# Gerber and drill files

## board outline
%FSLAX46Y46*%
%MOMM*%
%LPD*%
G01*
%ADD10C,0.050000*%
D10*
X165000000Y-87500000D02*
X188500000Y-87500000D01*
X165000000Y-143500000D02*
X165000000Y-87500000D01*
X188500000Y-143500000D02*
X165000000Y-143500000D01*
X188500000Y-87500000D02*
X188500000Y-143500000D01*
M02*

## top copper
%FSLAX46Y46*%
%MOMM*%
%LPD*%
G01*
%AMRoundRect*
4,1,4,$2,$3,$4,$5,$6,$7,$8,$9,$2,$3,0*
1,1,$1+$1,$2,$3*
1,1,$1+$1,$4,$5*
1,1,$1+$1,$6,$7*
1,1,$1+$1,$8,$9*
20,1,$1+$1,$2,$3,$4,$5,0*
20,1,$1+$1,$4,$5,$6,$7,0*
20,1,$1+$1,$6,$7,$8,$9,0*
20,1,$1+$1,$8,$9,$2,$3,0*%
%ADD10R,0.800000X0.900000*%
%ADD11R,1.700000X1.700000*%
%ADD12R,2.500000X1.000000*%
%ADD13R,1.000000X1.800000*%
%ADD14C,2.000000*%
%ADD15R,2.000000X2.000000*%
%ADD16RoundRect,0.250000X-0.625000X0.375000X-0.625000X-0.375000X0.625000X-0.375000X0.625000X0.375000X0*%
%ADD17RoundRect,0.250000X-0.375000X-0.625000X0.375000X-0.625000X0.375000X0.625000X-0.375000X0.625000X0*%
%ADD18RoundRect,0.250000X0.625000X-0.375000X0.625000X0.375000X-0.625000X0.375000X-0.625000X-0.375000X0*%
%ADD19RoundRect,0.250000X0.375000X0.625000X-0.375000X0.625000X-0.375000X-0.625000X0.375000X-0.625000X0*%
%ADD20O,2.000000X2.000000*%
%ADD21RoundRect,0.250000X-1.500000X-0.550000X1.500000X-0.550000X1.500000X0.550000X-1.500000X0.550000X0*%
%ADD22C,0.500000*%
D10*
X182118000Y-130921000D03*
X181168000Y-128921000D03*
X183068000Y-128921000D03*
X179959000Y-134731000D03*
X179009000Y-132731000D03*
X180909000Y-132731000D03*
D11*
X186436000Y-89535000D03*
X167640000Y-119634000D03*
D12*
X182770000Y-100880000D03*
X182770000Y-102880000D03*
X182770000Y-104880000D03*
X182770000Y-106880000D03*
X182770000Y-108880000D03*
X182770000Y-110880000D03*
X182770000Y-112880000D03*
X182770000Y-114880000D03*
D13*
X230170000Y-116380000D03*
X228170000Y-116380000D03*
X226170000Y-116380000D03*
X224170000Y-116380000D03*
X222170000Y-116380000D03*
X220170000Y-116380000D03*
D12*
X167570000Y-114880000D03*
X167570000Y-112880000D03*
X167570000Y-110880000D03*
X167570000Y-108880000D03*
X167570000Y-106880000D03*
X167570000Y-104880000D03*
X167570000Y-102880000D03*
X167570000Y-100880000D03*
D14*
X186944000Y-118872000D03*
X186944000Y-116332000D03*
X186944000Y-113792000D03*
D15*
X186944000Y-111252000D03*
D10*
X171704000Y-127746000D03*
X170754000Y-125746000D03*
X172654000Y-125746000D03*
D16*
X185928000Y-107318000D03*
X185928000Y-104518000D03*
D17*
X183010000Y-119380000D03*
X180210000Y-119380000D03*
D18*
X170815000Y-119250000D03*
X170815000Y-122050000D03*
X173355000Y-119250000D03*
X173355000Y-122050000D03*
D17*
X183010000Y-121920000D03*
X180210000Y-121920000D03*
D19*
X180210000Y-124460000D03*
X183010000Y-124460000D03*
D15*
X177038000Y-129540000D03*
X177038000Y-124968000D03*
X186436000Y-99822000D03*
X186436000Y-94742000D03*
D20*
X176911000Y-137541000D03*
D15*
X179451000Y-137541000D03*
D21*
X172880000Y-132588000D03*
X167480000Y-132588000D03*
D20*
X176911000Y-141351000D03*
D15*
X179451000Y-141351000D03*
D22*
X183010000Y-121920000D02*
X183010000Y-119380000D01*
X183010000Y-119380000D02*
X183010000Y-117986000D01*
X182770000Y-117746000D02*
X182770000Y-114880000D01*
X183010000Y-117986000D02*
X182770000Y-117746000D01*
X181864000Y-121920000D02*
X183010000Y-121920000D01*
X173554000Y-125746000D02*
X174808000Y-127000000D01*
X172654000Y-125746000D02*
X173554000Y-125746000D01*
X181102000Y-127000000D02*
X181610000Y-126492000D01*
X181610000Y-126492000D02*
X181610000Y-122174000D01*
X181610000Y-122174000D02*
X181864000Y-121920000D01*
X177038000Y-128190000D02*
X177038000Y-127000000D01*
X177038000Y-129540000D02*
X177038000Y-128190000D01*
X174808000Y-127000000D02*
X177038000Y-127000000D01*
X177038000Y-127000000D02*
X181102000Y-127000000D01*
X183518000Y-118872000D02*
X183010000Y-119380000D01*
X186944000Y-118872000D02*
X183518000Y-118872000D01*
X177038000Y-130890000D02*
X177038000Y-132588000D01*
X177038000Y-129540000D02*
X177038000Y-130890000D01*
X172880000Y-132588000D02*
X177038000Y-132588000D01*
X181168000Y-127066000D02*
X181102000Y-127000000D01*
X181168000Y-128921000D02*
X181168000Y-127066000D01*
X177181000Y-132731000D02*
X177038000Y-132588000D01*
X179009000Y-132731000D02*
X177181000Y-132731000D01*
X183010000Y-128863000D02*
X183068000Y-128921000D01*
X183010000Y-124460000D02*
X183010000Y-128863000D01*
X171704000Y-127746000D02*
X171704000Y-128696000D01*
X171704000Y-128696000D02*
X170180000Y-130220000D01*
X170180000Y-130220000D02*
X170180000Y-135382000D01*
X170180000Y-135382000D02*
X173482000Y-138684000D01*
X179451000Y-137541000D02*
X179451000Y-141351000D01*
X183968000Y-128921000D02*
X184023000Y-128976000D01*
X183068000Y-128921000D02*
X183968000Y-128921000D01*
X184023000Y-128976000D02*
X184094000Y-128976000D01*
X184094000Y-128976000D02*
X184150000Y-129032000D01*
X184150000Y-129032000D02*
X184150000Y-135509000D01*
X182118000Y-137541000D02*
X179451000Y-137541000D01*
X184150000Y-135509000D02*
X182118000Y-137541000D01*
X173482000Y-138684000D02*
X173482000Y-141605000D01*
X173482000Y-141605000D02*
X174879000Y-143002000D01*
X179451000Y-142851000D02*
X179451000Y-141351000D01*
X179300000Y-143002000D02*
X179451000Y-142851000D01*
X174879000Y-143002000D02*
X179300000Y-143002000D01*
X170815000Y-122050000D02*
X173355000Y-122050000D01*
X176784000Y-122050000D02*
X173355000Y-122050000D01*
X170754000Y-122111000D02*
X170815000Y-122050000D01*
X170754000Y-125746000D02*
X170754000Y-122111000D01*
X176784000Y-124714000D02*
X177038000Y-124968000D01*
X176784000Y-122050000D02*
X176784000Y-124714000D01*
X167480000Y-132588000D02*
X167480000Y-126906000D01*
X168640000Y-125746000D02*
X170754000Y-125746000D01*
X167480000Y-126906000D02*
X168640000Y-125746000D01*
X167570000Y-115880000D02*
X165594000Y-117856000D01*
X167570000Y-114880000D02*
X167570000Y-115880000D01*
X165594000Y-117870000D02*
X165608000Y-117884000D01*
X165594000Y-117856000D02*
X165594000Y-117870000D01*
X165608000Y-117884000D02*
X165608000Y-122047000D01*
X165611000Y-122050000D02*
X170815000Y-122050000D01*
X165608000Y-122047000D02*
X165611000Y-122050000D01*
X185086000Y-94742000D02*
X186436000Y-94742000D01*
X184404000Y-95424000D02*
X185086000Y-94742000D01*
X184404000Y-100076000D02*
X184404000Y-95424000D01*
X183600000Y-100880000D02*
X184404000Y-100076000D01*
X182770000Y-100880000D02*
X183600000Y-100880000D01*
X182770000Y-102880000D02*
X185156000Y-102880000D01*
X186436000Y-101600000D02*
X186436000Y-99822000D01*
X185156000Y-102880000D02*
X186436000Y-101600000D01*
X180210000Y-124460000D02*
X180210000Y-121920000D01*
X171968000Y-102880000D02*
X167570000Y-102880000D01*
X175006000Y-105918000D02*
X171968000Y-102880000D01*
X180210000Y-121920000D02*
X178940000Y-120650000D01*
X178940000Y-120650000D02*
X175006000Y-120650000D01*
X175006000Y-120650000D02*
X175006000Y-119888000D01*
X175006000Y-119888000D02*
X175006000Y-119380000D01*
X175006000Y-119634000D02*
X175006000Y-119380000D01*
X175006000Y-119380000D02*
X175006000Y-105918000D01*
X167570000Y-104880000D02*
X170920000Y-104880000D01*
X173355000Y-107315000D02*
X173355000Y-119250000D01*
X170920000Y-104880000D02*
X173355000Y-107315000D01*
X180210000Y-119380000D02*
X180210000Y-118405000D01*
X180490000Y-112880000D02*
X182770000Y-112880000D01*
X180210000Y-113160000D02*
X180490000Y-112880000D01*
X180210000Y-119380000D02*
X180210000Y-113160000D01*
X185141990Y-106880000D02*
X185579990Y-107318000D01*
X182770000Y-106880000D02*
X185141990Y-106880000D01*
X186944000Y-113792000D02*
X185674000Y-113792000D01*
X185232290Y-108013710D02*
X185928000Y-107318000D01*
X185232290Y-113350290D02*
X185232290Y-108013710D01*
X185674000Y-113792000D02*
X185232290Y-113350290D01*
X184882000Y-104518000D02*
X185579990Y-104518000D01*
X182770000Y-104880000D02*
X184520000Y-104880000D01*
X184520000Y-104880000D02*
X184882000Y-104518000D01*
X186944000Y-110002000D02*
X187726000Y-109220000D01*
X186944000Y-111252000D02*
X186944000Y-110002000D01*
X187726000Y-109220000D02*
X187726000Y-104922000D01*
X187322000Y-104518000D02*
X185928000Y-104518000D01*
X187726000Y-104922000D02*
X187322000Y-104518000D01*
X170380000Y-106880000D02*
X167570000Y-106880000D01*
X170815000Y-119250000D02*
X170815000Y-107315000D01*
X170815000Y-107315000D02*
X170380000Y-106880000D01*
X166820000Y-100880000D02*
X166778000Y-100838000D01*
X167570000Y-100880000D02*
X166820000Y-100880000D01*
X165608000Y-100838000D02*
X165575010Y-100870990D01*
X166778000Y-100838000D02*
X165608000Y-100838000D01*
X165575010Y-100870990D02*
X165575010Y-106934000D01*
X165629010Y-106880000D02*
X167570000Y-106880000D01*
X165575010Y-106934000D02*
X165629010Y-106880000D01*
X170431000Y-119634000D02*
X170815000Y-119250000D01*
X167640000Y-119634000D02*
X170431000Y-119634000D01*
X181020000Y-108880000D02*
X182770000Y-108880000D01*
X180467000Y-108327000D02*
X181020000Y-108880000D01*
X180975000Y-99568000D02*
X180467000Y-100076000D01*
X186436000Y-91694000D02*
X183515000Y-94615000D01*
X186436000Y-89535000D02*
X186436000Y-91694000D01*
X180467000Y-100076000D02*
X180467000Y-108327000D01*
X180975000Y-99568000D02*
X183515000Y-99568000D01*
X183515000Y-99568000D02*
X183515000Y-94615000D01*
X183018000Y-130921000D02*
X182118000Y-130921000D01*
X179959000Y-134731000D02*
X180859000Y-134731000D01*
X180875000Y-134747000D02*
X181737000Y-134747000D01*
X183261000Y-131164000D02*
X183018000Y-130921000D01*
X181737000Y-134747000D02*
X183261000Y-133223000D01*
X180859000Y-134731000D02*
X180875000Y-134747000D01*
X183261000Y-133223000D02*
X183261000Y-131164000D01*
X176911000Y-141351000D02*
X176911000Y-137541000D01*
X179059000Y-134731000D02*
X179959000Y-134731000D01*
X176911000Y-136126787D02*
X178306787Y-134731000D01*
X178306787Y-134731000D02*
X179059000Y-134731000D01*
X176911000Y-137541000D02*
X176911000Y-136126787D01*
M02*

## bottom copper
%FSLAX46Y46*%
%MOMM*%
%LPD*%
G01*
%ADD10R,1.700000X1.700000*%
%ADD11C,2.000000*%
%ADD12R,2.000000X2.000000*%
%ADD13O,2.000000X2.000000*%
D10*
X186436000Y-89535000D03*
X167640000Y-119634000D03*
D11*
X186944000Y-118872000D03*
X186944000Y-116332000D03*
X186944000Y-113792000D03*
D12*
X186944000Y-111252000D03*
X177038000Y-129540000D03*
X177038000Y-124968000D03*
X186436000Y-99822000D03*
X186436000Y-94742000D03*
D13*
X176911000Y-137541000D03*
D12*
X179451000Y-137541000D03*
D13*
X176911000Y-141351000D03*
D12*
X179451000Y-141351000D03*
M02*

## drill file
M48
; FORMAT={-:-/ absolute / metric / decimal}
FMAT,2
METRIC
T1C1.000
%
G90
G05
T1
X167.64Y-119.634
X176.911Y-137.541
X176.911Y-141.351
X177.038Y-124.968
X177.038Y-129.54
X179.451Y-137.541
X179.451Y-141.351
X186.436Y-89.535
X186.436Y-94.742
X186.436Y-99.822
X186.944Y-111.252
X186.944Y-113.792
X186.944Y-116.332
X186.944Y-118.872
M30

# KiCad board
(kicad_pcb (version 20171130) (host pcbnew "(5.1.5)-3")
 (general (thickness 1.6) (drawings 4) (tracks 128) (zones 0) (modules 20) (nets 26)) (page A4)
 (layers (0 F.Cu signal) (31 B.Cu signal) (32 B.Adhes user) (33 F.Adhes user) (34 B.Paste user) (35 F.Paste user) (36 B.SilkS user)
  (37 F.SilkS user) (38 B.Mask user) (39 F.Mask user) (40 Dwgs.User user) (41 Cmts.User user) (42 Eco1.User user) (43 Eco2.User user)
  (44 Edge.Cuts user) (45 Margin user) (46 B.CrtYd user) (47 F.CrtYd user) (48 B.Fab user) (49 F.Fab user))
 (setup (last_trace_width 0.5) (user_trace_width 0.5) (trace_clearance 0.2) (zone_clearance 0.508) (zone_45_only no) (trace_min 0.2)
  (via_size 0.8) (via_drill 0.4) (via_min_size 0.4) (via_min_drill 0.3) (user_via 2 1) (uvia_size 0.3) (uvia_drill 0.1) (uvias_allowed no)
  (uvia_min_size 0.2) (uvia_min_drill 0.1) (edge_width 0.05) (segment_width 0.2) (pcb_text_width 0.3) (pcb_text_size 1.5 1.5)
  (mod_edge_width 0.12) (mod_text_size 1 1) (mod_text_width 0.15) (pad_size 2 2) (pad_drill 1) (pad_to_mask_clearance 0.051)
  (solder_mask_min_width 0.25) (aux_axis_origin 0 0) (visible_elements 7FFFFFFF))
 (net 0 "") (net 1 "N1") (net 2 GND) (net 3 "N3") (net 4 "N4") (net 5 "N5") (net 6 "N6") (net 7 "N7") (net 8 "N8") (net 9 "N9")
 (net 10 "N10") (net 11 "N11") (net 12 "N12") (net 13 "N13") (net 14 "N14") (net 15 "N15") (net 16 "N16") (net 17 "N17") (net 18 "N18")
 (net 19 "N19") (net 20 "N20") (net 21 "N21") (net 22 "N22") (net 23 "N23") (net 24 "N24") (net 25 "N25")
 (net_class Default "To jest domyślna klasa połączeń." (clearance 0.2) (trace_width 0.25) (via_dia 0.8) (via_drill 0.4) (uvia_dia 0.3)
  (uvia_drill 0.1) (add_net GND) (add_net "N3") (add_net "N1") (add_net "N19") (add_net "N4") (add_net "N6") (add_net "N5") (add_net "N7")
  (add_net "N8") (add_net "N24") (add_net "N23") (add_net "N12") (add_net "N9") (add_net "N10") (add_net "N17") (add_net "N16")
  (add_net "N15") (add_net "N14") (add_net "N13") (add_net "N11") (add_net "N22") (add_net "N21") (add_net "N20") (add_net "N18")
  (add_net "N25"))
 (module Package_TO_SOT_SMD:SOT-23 (layer F.Cu) (at 182.118 129.921 270)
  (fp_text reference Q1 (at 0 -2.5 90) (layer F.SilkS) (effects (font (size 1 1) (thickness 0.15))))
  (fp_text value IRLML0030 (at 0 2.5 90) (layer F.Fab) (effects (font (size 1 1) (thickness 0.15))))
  (pad 3 smd rect (at 1 0 270) (size 0.9 0.8) (layers F.Cu F.Paste F.Mask) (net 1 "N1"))
  (pad 2 smd rect (at -1 0.95 270) (size 0.9 0.8) (layers F.Cu F.Paste F.Mask) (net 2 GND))
  (pad 1 smd rect (at -1 -0.95 270) (size 0.9 0.8) (layers F.Cu F.Paste F.Mask) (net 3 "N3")))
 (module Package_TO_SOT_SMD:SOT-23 (layer F.Cu) (at 179.959 133.731 270)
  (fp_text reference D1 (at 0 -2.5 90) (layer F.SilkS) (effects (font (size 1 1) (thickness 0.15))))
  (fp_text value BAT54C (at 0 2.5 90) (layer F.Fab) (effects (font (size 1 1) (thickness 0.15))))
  (pad 3 smd rect (at 1 0 270) (size 0.9 0.8) (layers F.Cu F.Paste F.Mask) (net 1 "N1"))
  (pad 2 smd rect (at -1 0.95 270) (size 0.9 0.8) (layers F.Cu F.Paste F.Mask) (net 2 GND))
  (pad 1 smd rect (at -1 -0.95 270) (size 0.9 0.8) (layers F.Cu F.Paste F.Mask) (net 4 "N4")))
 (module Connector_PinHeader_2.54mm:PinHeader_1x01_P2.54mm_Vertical (layer F.Cu) (at 186.436 89.535)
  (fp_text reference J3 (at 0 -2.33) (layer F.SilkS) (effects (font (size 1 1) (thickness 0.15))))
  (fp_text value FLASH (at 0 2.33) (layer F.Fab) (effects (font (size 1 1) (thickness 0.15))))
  (pad 1 thru_hole rect (at 0 0) (size 1.7 1.7) (drill 1) (layers *.Cu *.Mask) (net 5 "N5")))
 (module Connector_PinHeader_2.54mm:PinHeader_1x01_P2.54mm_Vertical (layer F.Cu) (at 167.64 119.634)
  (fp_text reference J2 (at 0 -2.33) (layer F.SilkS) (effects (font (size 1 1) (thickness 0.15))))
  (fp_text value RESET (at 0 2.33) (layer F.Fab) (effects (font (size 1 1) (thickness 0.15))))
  (pad 1 thru_hole rect (at 0 0) (size 1.7 1.7) (drill 1) (layers *.Cu *.Mask) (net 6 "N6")))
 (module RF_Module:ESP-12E (layer F.Cu) (at 175.17 104.38)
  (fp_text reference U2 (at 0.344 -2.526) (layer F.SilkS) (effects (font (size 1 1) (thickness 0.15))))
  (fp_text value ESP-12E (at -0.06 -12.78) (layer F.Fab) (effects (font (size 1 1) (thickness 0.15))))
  (pad 22 smd rect (at 7.6 -3.5) (size 2.5 1) (layers F.Cu F.Paste F.Mask) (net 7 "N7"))
  (pad 21 smd rect (at 7.6 -1.5) (size 2.5 1) (layers F.Cu F.Paste F.Mask) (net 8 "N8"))
  (pad 20 smd rect (at 7.6 0.5) (size 2.5 1) (layers F.Cu F.Paste F.Mask) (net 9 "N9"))
  (pad 19 smd rect (at 7.6 2.5) (size 2.5 1) (layers F.Cu F.Paste F.Mask) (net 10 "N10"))
  (pad 18 smd rect (at 7.6 4.5) (size 2.5 1) (layers F.Cu F.Paste F.Mask) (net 5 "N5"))
  (pad 17 smd rect (at 7.6 6.5) (size 2.5 1) (layers F.Cu F.Paste F.Mask) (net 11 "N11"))
  (pad 16 smd rect (at 7.6 8.5) (size 2.5 1) (layers F.Cu F.Paste F.Mask) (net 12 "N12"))
  (pad 15 smd rect (at 7.6 10.5) (size 2.5 1) (layers F.Cu F.Paste F.Mask) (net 2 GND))
  (pad 14 smd rect (at 55 12) (size 1 1.8) (layers F.Cu F.Paste F.Mask) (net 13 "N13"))
  (pad 13 smd rect (at 53 12) (size 1 1.8) (layers F.Cu F.Paste F.Mask) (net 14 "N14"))
  (pad 12 smd rect (at 51 12) (size 1 1.8) (layers F.Cu F.Paste F.Mask) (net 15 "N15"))
  (pad 11 smd rect (at 49 12) (size 1 1.8) (layers F.Cu F.Paste F.Mask) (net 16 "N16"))
  (pad 10 smd rect (at 47 12) (size 1 1.8) (layers F.Cu F.Paste F.Mask) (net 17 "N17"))
  (pad 9 smd rect (at 45 12) (size 1 1.8) (layers F.Cu F.Paste F.Mask) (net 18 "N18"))
  (pad 8 smd rect (at -7.6 10.5) (size 2.5 1) (layers F.Cu F.Paste F.Mask) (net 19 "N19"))
  (pad 7 smd rect (at -7.6 8.5) (size 2.5 1) (layers F.Cu F.Paste F.Mask) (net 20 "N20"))
  (pad 6 smd rect (at -7.6 6.5) (size 2.5 1) (layers F.Cu F.Paste F.Mask) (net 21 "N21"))
  (pad 5 smd rect (at -7.6 4.5) (size 2.5 1) (layers F.Cu F.Paste F.Mask) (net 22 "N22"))
  (pad 4 smd rect (at -7.6 2.5) (size 2.5 1) (layers F.Cu F.Paste F.Mask) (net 6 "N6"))
  (pad 3 smd rect (at -7.6 0.5) (size 2.5 1) (layers F.Cu F.Paste F.Mask) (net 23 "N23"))
  (pad 2 smd rect (at -7.6 -1.5) (size 2.5 1) (layers F.Cu F.Paste F.Mask) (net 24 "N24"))
  (pad 1 smd rect (at -7.6 -3.5) (size 2.5 1) (layers F.Cu F.Paste F.Mask) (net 6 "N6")))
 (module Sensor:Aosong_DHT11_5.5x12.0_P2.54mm (layer F.Cu) (at 186.944 111.252)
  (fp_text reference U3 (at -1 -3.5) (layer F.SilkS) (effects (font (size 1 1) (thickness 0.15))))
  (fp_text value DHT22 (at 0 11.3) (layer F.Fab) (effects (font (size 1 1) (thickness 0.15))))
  (pad 4 thru_hole circle (at 0 7.62) (size 2 2) (drill 1) (layers *.Cu *.Mask) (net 2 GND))
  (pad 3 thru_hole circle (at 0 5.08) (size 2 2) (drill 1) (layers *.Cu *.Mask) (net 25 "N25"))
  (pad 2 thru_hole circle (at 0 2.54) (size 2 2) (drill 1) (layers *.Cu *.Mask) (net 10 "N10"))
  (pad 1 thru_hole rect (at 0 0) (size 2 2) (drill 1) (layers *.Cu *.Mask) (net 9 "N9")))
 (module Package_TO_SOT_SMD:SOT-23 (layer F.Cu) (at 171.704 126.746 270)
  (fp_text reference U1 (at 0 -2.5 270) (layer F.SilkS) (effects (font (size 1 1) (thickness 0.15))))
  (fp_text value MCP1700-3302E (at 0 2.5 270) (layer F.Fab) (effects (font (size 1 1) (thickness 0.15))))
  (pad 3 smd rect (at 1 0 270) (size 0.9 0.8) (layers F.Cu F.Paste F.Mask) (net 3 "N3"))
  (pad 2 smd rect (at -1 0.95 270) (size 0.9 0.8) (layers F.Cu F.Paste F.Mask) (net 19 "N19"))
  (pad 1 smd rect (at -1 -0.95 270) (size 0.9 0.8) (layers F.Cu F.Paste F.Mask) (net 2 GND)))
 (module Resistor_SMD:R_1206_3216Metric (layer F.Cu) (at 185.928 105.918 270)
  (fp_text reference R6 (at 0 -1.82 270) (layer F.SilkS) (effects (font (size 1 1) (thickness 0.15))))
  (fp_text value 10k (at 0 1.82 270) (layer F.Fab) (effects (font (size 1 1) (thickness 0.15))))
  (pad 2 smd roundrect (at 1.4 0 270) (size 1.25 1.75) (layers F.Cu F.Paste F.Mask) (roundrect_rratio 0.2) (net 10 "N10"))
  (pad 1 smd roundrect (at -1.4 0 270) (size 1.25 1.75) (layers F.Cu F.Paste F.Mask) (roundrect_rratio 0.2) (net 9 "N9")))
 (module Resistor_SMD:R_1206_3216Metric (layer F.Cu) (at 181.61 119.38)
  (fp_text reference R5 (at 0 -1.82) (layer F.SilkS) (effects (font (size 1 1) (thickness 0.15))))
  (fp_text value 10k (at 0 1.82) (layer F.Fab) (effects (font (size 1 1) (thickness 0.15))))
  (pad 2 smd roundrect (at 1.4 0) (size 1.25 1.75) (layers F.Cu F.Paste F.Mask) (roundrect_rratio 0.2) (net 2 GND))
  (pad 1 smd roundrect (at -1.4 0) (size 1.25 1.75) (layers F.Cu F.Paste F.Mask) (roundrect_rratio 0.2) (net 12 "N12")))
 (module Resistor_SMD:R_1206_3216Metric (layer F.Cu) (at 170.815 120.65 90)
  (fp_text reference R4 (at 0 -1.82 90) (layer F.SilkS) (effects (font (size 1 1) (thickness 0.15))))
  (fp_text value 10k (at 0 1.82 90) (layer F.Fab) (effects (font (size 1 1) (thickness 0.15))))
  (pad 2 smd roundrect (at 1.4 0 90) (size 1.25 1.75) (layers F.Cu F.Paste F.Mask) (roundrect_rratio 0.2) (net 6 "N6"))
  (pad 1 smd roundrect (at -1.4 0 90) (size 1.25 1.75) (layers F.Cu F.Paste F.Mask) (roundrect_rratio 0.2) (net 19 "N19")))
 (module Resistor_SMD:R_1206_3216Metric (layer F.Cu) (at 173.355 120.65 90)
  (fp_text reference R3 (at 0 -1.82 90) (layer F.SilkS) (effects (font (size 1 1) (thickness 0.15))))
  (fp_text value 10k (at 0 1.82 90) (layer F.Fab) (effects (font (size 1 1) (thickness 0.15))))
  (pad 2 smd roundrect (at 1.4 0 90) (size 1.25 1.75) (layers F.Cu F.Paste F.Mask) (roundrect_rratio 0.2) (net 23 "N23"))
  (pad 1 smd roundrect (at -1.4 0 90) (size 1.25 1.75) (layers F.Cu F.Paste F.Mask) (roundrect_rratio 0.2) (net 19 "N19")))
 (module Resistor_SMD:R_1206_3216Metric (layer F.Cu) (at 181.61 121.92)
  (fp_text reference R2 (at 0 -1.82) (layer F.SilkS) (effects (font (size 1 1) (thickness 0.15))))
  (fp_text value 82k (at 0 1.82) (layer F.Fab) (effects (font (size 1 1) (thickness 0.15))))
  (pad 2 smd roundrect (at 1.4 0) (size 1.25 1.75) (layers F.Cu F.Paste F.Mask) (roundrect_rratio 0.2) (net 2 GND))
  (pad 1 smd roundrect (at -1.4 0) (size 1.25 1.75) (layers F.Cu F.Paste F.Mask) (roundrect_rratio 0.2) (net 24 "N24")))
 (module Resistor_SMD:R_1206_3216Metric (layer F.Cu) (at 181.61 124.46 180)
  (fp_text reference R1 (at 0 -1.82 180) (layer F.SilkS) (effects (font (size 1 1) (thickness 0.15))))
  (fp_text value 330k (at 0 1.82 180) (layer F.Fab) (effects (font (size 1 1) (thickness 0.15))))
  (pad 2 smd roundrect (at 1.4 0 180) (size 1.25 1.75) (layers F.Cu F.Paste F.Mask) (roundrect_rratio 0.2) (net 24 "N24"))
  (pad 1 smd roundrect (at -1.4 0 180) (size 1.25 1.75) (layers F.Cu F.Paste F.Mask) (roundrect_rratio 0.2) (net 3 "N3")))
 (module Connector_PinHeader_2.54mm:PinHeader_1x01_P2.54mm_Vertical (layer F.Cu) (at 177.038 129.54)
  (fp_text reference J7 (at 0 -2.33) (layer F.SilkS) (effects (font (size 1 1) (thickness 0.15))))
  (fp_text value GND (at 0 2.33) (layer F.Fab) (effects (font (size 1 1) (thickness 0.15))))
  (pad 1 thru_hole rect (at 0 0) (size 2 2) (drill 1) (layers *.Cu *.Mask) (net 2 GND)))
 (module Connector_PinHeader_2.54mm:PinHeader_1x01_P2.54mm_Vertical (layer F.Cu) (at 177.038 124.968)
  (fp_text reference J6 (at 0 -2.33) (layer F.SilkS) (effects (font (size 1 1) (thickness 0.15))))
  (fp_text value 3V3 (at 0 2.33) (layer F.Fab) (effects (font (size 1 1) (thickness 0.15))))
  (pad 1 thru_hole rect (at 0 0) (size 2 2) (drill 1) (layers *.Cu *.Mask) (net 19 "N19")))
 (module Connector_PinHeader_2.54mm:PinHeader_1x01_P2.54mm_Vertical (layer F.Cu) (at 186.436 99.822)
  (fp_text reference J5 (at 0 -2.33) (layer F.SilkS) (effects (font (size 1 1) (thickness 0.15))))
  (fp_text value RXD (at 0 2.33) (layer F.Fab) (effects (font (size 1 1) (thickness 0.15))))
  (pad 1 thru_hole rect (at 0 0) (size 2 2) (drill 1) (layers *.Cu *.Mask) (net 8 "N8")))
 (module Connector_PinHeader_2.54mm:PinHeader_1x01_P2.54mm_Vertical (layer F.Cu) (at 186.436 94.742)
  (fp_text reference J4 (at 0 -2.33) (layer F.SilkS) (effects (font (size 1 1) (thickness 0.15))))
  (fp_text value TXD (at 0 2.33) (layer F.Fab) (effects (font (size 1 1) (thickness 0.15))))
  (pad 1 thru_hole rect (at 0 0) (size 2 2) (drill 1) (layers *.Cu *.Mask) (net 7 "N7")))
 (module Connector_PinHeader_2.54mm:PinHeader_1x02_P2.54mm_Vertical (layer F.Cu) (at 179.451 137.541 270)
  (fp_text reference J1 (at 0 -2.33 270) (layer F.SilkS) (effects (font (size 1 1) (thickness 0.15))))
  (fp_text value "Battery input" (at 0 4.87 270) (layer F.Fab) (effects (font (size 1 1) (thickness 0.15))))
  (pad 2 thru_hole oval (at 0 2.54 270) (size 2 2) (drill 1) (layers *.Cu *.Mask) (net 1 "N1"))
  (pad 1 thru_hole rect (at 0 0 270) (size 2 2) (drill 1) (layers *.Cu *.Mask) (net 3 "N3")))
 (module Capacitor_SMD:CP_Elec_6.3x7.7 (layer F.Cu) (at 170.18 132.588)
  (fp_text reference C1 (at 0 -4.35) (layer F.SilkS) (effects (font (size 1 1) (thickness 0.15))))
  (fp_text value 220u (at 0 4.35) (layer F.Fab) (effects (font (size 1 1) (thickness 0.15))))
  (pad 2 smd roundrect (at 2.7 0) (size 3.5 1.6) (layers F.Cu F.Paste F.Mask) (roundrect_rratio 0.15625) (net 2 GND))
  (pad 1 smd roundrect (at -2.7 0) (size 3.5 1.6) (layers F.Cu F.Paste F.Mask) (roundrect_rratio 0.15625) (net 19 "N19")))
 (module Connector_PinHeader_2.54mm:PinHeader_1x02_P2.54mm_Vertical (layer F.Cu) (at 179.451 141.351 270)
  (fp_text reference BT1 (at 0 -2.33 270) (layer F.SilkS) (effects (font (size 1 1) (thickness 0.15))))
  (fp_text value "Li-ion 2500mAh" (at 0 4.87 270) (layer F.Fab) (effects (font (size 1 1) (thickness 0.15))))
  (pad 2 thru_hole oval (at 0 2.54 270) (size 2 2) (drill 1) (layers *.Cu *.Mask) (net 1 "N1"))
  (pad 1 thru_hole rect (at 0 0 270) (size 2 2) (drill 1) (layers *.Cu *.Mask) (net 3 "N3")))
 (gr_line (start 165 87.5) (end 188.5 87.5) (layer Edge.Cuts) (width 0.05))
 (gr_line (start 165 143.5) (end 165 87.5) (layer Edge.Cuts) (width 0.05))
 (gr_line (start 188.5 143.5) (end 165 143.5) (layer Edge.Cuts) (width 0.05))
 (gr_line (start 188.5 87.5) (end 188.5 143.5) (layer Edge.Cuts) (width 0.05))
 (segment (start 183.01 121.92) (end 183.01 119.38) (width 0.5) (layer F.Cu) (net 2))
 (segment (start 183.01 119.38) (end 183.01 117.986) (width 0.5) (layer F.Cu) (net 2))
 (segment (start 182.77 117.746) (end 182.77 114.88) (width 0.5) (layer F.Cu) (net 2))
 (segment (start 183.01 117.986) (end 182.77 117.746) (width 0.5) (layer F.Cu) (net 2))
 (segment (start 181.864 121.92) (end 183.01 121.92) (width 0.5) (layer F.Cu) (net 2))
 (segment (start 173.554 125.746) (end 174.808 127) (width 0.5) (layer F.Cu) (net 2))
 (segment (start 172.654 125.746) (end 173.554 125.746) (width 0.5) (layer F.Cu) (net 2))
 (segment (start 181.102 127) (end 181.61 126.492) (width 0.5) (layer F.Cu) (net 2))
 (segment (start 181.61 126.492) (end 181.61 122.174) (width 0.5) (layer F.Cu) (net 2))
 (segment (start 181.61 122.174) (end 181.864 121.92) (width 0.5) (layer F.Cu) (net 2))
 (segment (start 177.038 128.19) (end 177.038 127) (width 0.5) (layer F.Cu) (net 2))
 (segment (start 177.038 129.54) (end 177.038 128.19) (width 0.5) (layer F.Cu) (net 2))
 (segment (start 174.808 127) (end 177.038 127) (width 0.5) (layer F.Cu) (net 2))
 (segment (start 177.038 127) (end 181.102 127) (width 0.5) (layer F.Cu) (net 2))
 (segment (start 183.518 118.872) (end 183.01 119.38) (width 0.5) (layer F.Cu) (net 2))
 (segment (start 186.944 118.872) (end 183.518 118.872) (width 0.5) (layer F.Cu) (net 2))
 (segment (start 177.038 130.89) (end 177.038 132.588) (width 0.5) (layer F.Cu) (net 2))
 (segment (start 177.038 129.54) (end 177.038 130.89) (width 0.5) (layer F.Cu) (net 2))
 (segment (start 172.88 132.588) (end 177.038 132.588) (width 0.5) (layer F.Cu) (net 2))
 (segment (start 181.168 127.066) (end 181.102 127) (width 0.5) (layer F.Cu) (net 2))
 (segment (start 181.168 128.921) (end 181.168 127.066) (width 0.5) (layer F.Cu) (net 2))
 (segment (start 177.181 132.731) (end 177.038 132.588) (width 0.5) (layer F.Cu) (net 2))
 (segment (start 179.009 132.731) (end 177.181 132.731) (width 0.5) (layer F.Cu) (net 2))
 (segment (start 183.01 128.863) (end 183.068 128.921) (width 0.5) (layer F.Cu) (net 3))
 (segment (start 183.01 124.46) (end 183.01 128.863) (width 0.5) (layer F.Cu) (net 3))
 (segment (start 171.704 127.746) (end 171.704 128.696) (width 0.5) (layer F.Cu) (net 3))
 (segment (start 171.704 128.696) (end 170.18 130.22) (width 0.5) (layer F.Cu) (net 3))
 (segment (start 170.18 130.22) (end 170.18 135.382) (width 0.5) (layer F.Cu) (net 3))
 (segment (start 170.18 135.382) (end 173.482 138.684) (width 0.5) (layer F.Cu) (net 3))
 (segment (start 179.451 137.541) (end 179.451 141.351) (width 0.5) (layer F.Cu) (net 3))
 (segment (start 183.968 128.921) (end 184.023 128.976) (width 0.5) (layer F.Cu) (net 3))
 (segment (start 183.068 128.921) (end 183.968 128.921) (width 0.5) (layer F.Cu) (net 3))
 (segment (start 184.023 128.976) (end 184.094 128.976) (width 0.5) (layer F.Cu) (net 3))
 (segment (start 184.094 128.976) (end 184.15 129.032) (width 0.5) (layer F.Cu) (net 3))
 (segment (start 184.15 129.032) (end 184.15 135.509) (width 0.5) (layer F.Cu) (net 3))
 (segment (start 182.118 137.541) (end 179.451 137.541) (width 0.5) (layer F.Cu) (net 3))
 (segment (start 184.15 135.509) (end 182.118 137.541) (width 0.5) (layer F.Cu) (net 3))
 (segment (start 173.482 138.684) (end 173.482 141.605) (width 0.5) (layer F.Cu) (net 3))
 (segment (start 173.482 141.605) (end 174.879 143.002) (width 0.5) (layer F.Cu) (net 3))
 (segment (start 179.451 142.851) (end 179.451 141.351) (width 0.5) (layer F.Cu) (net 3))
 (segment (start 179.3 143.002) (end 179.451 142.851) (width 0.5) (layer F.Cu) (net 3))
 (segment (start 174.879 143.002) (end 179.3 143.002) (width 0.5) (layer F.Cu) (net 3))
 (segment (start 170.815 122.05) (end 173.355 122.05) (width 0.5) (layer F.Cu) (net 19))
 (segment (start 176.784 122.05) (end 173.355 122.05) (width 0.5) (layer F.Cu) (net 19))
 (segment (start 170.754 122.111) (end 170.815 122.05) (width 0.5) (layer F.Cu) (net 19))
 (segment (start 170.754 125.746) (end 170.754 122.111) (width 0.5) (layer F.Cu) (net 19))
 (segment (start 176.784 124.714) (end 177.038 124.968) (width 0.5) (layer F.Cu) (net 19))
 (segment (start 176.784 122.05) (end 176.784 124.714) (width 0.5) (layer F.Cu) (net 19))
 (segment (start 167.48 132.588) (end 167.48 126.906) (width 0.5) (layer F.Cu) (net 19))
 (segment (start 168.64 125.746) (end 170.754 125.746) (width 0.5) (layer F.Cu) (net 19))
 (segment (start 167.48 126.906) (end 168.64 125.746) (width 0.5) (layer F.Cu) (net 19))
 (segment (start 167.57 115.88) (end 165.594 117.856) (width 0.5) (layer F.Cu) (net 19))
 (segment (start 167.57 114.88) (end 167.57 115.88) (width 0.5) (layer F.Cu) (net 19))
 (segment (start 165.594 117.87) (end 165.608 117.884) (width 0.5) (layer F.Cu) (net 19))
 (segment (start 165.594 117.856) (end 165.594 117.87) (width 0.5) (layer F.Cu) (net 19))
 (segment (start 165.608 117.884) (end 165.608 122.047) (width 0.5) (layer F.Cu) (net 19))
 (segment (start 165.611 122.05) (end 170.815 122.05) (width 0.5) (layer F.Cu) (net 19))
 (segment (start 165.608 122.047) (end 165.611 122.05) (width 0.5) (layer F.Cu) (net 19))
 (segment (start 185.086 94.742) (end 186.436 94.742) (width 0.5) (layer F.Cu) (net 7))
 (segment (start 184.404 95.424) (end 185.086 94.742) (width 0.5) (layer F.Cu) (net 7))
 (segment (start 184.404 100.076) (end 184.404 95.424) (width 0.5) (layer F.Cu) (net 7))
 (segment (start 183.6 100.88) (end 184.404 100.076) (width 0.5) (layer F.Cu) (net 7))
 (segment (start 182.77 100.88) (end 183.6 100.88) (width 0.5) (layer F.Cu) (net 7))
 (segment (start 182.77 102.88) (end 185.156 102.88) (width 0.5) (layer F.Cu) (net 8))
 (segment (start 186.436 101.6) (end 186.436 99.822) (width 0.5) (layer F.Cu) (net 8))
 (segment (start 185.156 102.88) (end 186.436 101.6) (width 0.5) (layer F.Cu) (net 8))
 (segment (start 180.21 124.46) (end 180.21 121.92) (width 0.5) (layer F.Cu) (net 24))
 (segment (start 171.968 102.88) (end 167.57 102.88) (width 0.5) (layer F.Cu) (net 24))
 (segment (start 175.006 105.918) (end 171.968 102.88) (width 0.5) (layer F.Cu) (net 24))
 (segment (start 180.21 121.92) (end 178.94 120.65) (width 0.5) (layer F.Cu) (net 24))
 (segment (start 178.94 120.65) (end 175.006 120.65) (width 0.5) (layer F.Cu) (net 24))
 (segment (start 175.006 120.65) (end 175.006 119.888) (width 0.5) (layer F.Cu) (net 24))
 (segment (start 175.006 119.888) (end 175.006 119.38) (width 0.5) (layer F.Cu) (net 24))
 (segment (start 175.006 119.634) (end 175.006 119.38) (width 0.5) (layer F.Cu) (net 24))
 (segment (start 175.006 119.38) (end 175.006 105.918) (width 0.5) (layer F.Cu) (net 24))
 (segment (start 167.57 104.88) (end 170.92 104.88) (width 0.5) (layer F.Cu) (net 23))
 (segment (start 173.355 107.315) (end 173.355 119.25) (width 0.5) (layer F.Cu) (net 23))
 (segment (start 170.92 104.88) (end 173.355 107.315) (width 0.5) (layer F.Cu) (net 23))
 (segment (start 180.21 119.38) (end 180.21 118.405) (width 0.5) (layer F.Cu) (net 12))
 (segment (start 180.49 112.88) (end 182.77 112.88) (width 0.5) (layer F.Cu) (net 12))
 (segment (start 180.21 113.16) (end 180.49 112.88) (width 0.5) (layer F.Cu) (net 12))
 (segment (start 180.21 119.38) (end 180.21 113.16) (width 0.5) (layer F.Cu) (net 12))
 (segment (start 185.14199 106.88) (end 185.57999 107.318) (width 0.5) (layer F.Cu) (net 10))
 (segment (start 182.77 106.88) (end 185.14199 106.88) (width 0.5) (layer F.Cu) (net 10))
 (segment (start 186.944 113.792) (end 185.674 113.792) (width 0.5) (layer F.Cu) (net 10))
 (segment (start 185.23229 108.01371) (end 185.928 107.318) (width 0.5) (layer F.Cu) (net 10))
 (segment (start 185.23229 113.35029) (end 185.23229 108.01371) (width 0.5) (layer F.Cu) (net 10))
 (segment (start 185.674 113.792) (end 185.23229 113.35029) (width 0.5) (layer F.Cu) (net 10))
 (segment (start 184.882 104.518) (end 185.57999 104.518) (width 0.5) (layer F.Cu) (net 9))
 (segment (start 182.77 104.88) (end 184.52 104.88) (width 0.5) (layer F.Cu) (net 9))
 (segment (start 184.52 104.88) (end 184.882 104.518) (width 0.5) (layer F.Cu) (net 9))
 (segment (start 186.944 110.002) (end 187.726 109.22) (width 0.5) (layer F.Cu) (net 9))
 (segment (start 186.944 111.252) (end 186.944 110.002) (width 0.5) (layer F.Cu) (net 9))
 (segment (start 187.726 109.22) (end 187.726 104.922) (width 0.5) (layer F.Cu) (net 9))
 (segment (start 187.322 104.518) (end 185.928 104.518) (width 0.5) (layer F.Cu) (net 9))
 (segment (start 187.726 104.922) (end 187.322 104.518) (width 0.5) (layer F.Cu) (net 9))
 (segment (start 170.38 106.88) (end 167.57 106.88) (width 0.5) (layer F.Cu) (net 6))
 (segment (start 170.815 119.25) (end 170.815 107.315) (width 0.5) (layer F.Cu) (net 6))
 (segment (start 170.815 107.315) (end 170.38 106.88) (width 0.5) (layer F.Cu) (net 6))
 (segment (start 166.82 100.88) (end 166.778 100.838) (width 0.5) (layer F.Cu) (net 6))
 (segment (start 167.57 100.88) (end 166.82 100.88) (width 0.5) (layer F.Cu) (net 6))
 (segment (start 165.608 100.838) (end 165.57501 100.87099) (width 0.5) (layer F.Cu) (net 6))
 (segment (start 166.778 100.838) (end 165.608 100.838) (width 0.5) (layer F.Cu) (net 6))
 (segment (start 165.57501 100.87099) (end 165.57501 106.934) (width 0.5) (layer F.Cu) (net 6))
 (segment (start 165.62901 106.88) (end 167.57 106.88) (width 0.5) (layer F.Cu) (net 6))
 (segment (start 165.57501 106.934) (end 165.62901 106.88) (width 0.5) (layer F.Cu) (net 6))
 (segment (start 170.431 119.634) (end 170.815 119.25) (width 0.5) (layer F.Cu) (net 6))
 (segment (start 167.64 119.634) (end 170.431 119.634) (width 0.5) (layer F.Cu) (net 6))
 (segment (start 181.02 108.88) (end 182.77 108.88) (width 0.5) (layer F.Cu) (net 5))
 (segment (start 180.467 108.327) (end 181.02 108.88) (width 0.5) (layer F.Cu) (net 5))
 (segment (start 180.975 99.568) (end 180.467 100.076) (width 0.5) (layer F.Cu) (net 5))
 (segment (start 186.436 91.694) (end 183.515 94.615) (width 0.5) (layer F.Cu) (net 5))
 (segment (start 186.436 89.535) (end 186.436 91.694) (width 0.5) (layer F.Cu) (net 5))
 (segment (start 180.467 100.076) (end 180.467 108.327) (width 0.5) (layer F.Cu) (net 5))
 (segment (start 180.975 99.568) (end 183.515 99.568) (width 0.5) (layer F.Cu) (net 5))
 (segment (start 183.515 99.568) (end 183.515 94.615) (width 0.5) (layer F.Cu) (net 5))
 (segment (start 183.018 130.921) (end 182.118 130.921) (width 0.5) (layer F.Cu) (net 1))
 (segment (start 179.959 134.731) (end 180.859 134.731) (width 0.5) (layer F.Cu) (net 1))
 (segment (start 180.875 134.747) (end 181.737 134.747) (width 0.5) (layer F.Cu) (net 1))
 (segment (start 183.261 131.164) (end 183.018 130.921) (width 0.5) (layer F.Cu) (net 1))
 (segment (start 181.737 134.747) (end 183.261 133.223) (width 0.5) (layer F.Cu) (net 1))
 (segment (start 180.859 134.731) (end 180.875 134.747) (width 0.5) (layer F.Cu) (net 1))
 (segment (start 183.261 133.223) (end 183.261 131.164) (width 0.5) (layer F.Cu) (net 1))
 (segment (start 176.911 141.351) (end 176.911 137.541) (width 0.5) (layer F.Cu) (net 1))
 (segment (start 179.059 134.731) (end 179.959 134.731) (width 0.5) (layer F.Cu) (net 1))
 (segment (start 176.911 136.126787) (end 178.306787 134.731) (width 0.5) (layer F.Cu) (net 1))
 (segment (start 178.306787 134.731) (end 179.059 134.731) (width 0.5) (layer F.Cu) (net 1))
 (segment (start 176.911 137.541) (end 176.911 136.126787) (width 0.5) (layer F.Cu) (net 1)))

